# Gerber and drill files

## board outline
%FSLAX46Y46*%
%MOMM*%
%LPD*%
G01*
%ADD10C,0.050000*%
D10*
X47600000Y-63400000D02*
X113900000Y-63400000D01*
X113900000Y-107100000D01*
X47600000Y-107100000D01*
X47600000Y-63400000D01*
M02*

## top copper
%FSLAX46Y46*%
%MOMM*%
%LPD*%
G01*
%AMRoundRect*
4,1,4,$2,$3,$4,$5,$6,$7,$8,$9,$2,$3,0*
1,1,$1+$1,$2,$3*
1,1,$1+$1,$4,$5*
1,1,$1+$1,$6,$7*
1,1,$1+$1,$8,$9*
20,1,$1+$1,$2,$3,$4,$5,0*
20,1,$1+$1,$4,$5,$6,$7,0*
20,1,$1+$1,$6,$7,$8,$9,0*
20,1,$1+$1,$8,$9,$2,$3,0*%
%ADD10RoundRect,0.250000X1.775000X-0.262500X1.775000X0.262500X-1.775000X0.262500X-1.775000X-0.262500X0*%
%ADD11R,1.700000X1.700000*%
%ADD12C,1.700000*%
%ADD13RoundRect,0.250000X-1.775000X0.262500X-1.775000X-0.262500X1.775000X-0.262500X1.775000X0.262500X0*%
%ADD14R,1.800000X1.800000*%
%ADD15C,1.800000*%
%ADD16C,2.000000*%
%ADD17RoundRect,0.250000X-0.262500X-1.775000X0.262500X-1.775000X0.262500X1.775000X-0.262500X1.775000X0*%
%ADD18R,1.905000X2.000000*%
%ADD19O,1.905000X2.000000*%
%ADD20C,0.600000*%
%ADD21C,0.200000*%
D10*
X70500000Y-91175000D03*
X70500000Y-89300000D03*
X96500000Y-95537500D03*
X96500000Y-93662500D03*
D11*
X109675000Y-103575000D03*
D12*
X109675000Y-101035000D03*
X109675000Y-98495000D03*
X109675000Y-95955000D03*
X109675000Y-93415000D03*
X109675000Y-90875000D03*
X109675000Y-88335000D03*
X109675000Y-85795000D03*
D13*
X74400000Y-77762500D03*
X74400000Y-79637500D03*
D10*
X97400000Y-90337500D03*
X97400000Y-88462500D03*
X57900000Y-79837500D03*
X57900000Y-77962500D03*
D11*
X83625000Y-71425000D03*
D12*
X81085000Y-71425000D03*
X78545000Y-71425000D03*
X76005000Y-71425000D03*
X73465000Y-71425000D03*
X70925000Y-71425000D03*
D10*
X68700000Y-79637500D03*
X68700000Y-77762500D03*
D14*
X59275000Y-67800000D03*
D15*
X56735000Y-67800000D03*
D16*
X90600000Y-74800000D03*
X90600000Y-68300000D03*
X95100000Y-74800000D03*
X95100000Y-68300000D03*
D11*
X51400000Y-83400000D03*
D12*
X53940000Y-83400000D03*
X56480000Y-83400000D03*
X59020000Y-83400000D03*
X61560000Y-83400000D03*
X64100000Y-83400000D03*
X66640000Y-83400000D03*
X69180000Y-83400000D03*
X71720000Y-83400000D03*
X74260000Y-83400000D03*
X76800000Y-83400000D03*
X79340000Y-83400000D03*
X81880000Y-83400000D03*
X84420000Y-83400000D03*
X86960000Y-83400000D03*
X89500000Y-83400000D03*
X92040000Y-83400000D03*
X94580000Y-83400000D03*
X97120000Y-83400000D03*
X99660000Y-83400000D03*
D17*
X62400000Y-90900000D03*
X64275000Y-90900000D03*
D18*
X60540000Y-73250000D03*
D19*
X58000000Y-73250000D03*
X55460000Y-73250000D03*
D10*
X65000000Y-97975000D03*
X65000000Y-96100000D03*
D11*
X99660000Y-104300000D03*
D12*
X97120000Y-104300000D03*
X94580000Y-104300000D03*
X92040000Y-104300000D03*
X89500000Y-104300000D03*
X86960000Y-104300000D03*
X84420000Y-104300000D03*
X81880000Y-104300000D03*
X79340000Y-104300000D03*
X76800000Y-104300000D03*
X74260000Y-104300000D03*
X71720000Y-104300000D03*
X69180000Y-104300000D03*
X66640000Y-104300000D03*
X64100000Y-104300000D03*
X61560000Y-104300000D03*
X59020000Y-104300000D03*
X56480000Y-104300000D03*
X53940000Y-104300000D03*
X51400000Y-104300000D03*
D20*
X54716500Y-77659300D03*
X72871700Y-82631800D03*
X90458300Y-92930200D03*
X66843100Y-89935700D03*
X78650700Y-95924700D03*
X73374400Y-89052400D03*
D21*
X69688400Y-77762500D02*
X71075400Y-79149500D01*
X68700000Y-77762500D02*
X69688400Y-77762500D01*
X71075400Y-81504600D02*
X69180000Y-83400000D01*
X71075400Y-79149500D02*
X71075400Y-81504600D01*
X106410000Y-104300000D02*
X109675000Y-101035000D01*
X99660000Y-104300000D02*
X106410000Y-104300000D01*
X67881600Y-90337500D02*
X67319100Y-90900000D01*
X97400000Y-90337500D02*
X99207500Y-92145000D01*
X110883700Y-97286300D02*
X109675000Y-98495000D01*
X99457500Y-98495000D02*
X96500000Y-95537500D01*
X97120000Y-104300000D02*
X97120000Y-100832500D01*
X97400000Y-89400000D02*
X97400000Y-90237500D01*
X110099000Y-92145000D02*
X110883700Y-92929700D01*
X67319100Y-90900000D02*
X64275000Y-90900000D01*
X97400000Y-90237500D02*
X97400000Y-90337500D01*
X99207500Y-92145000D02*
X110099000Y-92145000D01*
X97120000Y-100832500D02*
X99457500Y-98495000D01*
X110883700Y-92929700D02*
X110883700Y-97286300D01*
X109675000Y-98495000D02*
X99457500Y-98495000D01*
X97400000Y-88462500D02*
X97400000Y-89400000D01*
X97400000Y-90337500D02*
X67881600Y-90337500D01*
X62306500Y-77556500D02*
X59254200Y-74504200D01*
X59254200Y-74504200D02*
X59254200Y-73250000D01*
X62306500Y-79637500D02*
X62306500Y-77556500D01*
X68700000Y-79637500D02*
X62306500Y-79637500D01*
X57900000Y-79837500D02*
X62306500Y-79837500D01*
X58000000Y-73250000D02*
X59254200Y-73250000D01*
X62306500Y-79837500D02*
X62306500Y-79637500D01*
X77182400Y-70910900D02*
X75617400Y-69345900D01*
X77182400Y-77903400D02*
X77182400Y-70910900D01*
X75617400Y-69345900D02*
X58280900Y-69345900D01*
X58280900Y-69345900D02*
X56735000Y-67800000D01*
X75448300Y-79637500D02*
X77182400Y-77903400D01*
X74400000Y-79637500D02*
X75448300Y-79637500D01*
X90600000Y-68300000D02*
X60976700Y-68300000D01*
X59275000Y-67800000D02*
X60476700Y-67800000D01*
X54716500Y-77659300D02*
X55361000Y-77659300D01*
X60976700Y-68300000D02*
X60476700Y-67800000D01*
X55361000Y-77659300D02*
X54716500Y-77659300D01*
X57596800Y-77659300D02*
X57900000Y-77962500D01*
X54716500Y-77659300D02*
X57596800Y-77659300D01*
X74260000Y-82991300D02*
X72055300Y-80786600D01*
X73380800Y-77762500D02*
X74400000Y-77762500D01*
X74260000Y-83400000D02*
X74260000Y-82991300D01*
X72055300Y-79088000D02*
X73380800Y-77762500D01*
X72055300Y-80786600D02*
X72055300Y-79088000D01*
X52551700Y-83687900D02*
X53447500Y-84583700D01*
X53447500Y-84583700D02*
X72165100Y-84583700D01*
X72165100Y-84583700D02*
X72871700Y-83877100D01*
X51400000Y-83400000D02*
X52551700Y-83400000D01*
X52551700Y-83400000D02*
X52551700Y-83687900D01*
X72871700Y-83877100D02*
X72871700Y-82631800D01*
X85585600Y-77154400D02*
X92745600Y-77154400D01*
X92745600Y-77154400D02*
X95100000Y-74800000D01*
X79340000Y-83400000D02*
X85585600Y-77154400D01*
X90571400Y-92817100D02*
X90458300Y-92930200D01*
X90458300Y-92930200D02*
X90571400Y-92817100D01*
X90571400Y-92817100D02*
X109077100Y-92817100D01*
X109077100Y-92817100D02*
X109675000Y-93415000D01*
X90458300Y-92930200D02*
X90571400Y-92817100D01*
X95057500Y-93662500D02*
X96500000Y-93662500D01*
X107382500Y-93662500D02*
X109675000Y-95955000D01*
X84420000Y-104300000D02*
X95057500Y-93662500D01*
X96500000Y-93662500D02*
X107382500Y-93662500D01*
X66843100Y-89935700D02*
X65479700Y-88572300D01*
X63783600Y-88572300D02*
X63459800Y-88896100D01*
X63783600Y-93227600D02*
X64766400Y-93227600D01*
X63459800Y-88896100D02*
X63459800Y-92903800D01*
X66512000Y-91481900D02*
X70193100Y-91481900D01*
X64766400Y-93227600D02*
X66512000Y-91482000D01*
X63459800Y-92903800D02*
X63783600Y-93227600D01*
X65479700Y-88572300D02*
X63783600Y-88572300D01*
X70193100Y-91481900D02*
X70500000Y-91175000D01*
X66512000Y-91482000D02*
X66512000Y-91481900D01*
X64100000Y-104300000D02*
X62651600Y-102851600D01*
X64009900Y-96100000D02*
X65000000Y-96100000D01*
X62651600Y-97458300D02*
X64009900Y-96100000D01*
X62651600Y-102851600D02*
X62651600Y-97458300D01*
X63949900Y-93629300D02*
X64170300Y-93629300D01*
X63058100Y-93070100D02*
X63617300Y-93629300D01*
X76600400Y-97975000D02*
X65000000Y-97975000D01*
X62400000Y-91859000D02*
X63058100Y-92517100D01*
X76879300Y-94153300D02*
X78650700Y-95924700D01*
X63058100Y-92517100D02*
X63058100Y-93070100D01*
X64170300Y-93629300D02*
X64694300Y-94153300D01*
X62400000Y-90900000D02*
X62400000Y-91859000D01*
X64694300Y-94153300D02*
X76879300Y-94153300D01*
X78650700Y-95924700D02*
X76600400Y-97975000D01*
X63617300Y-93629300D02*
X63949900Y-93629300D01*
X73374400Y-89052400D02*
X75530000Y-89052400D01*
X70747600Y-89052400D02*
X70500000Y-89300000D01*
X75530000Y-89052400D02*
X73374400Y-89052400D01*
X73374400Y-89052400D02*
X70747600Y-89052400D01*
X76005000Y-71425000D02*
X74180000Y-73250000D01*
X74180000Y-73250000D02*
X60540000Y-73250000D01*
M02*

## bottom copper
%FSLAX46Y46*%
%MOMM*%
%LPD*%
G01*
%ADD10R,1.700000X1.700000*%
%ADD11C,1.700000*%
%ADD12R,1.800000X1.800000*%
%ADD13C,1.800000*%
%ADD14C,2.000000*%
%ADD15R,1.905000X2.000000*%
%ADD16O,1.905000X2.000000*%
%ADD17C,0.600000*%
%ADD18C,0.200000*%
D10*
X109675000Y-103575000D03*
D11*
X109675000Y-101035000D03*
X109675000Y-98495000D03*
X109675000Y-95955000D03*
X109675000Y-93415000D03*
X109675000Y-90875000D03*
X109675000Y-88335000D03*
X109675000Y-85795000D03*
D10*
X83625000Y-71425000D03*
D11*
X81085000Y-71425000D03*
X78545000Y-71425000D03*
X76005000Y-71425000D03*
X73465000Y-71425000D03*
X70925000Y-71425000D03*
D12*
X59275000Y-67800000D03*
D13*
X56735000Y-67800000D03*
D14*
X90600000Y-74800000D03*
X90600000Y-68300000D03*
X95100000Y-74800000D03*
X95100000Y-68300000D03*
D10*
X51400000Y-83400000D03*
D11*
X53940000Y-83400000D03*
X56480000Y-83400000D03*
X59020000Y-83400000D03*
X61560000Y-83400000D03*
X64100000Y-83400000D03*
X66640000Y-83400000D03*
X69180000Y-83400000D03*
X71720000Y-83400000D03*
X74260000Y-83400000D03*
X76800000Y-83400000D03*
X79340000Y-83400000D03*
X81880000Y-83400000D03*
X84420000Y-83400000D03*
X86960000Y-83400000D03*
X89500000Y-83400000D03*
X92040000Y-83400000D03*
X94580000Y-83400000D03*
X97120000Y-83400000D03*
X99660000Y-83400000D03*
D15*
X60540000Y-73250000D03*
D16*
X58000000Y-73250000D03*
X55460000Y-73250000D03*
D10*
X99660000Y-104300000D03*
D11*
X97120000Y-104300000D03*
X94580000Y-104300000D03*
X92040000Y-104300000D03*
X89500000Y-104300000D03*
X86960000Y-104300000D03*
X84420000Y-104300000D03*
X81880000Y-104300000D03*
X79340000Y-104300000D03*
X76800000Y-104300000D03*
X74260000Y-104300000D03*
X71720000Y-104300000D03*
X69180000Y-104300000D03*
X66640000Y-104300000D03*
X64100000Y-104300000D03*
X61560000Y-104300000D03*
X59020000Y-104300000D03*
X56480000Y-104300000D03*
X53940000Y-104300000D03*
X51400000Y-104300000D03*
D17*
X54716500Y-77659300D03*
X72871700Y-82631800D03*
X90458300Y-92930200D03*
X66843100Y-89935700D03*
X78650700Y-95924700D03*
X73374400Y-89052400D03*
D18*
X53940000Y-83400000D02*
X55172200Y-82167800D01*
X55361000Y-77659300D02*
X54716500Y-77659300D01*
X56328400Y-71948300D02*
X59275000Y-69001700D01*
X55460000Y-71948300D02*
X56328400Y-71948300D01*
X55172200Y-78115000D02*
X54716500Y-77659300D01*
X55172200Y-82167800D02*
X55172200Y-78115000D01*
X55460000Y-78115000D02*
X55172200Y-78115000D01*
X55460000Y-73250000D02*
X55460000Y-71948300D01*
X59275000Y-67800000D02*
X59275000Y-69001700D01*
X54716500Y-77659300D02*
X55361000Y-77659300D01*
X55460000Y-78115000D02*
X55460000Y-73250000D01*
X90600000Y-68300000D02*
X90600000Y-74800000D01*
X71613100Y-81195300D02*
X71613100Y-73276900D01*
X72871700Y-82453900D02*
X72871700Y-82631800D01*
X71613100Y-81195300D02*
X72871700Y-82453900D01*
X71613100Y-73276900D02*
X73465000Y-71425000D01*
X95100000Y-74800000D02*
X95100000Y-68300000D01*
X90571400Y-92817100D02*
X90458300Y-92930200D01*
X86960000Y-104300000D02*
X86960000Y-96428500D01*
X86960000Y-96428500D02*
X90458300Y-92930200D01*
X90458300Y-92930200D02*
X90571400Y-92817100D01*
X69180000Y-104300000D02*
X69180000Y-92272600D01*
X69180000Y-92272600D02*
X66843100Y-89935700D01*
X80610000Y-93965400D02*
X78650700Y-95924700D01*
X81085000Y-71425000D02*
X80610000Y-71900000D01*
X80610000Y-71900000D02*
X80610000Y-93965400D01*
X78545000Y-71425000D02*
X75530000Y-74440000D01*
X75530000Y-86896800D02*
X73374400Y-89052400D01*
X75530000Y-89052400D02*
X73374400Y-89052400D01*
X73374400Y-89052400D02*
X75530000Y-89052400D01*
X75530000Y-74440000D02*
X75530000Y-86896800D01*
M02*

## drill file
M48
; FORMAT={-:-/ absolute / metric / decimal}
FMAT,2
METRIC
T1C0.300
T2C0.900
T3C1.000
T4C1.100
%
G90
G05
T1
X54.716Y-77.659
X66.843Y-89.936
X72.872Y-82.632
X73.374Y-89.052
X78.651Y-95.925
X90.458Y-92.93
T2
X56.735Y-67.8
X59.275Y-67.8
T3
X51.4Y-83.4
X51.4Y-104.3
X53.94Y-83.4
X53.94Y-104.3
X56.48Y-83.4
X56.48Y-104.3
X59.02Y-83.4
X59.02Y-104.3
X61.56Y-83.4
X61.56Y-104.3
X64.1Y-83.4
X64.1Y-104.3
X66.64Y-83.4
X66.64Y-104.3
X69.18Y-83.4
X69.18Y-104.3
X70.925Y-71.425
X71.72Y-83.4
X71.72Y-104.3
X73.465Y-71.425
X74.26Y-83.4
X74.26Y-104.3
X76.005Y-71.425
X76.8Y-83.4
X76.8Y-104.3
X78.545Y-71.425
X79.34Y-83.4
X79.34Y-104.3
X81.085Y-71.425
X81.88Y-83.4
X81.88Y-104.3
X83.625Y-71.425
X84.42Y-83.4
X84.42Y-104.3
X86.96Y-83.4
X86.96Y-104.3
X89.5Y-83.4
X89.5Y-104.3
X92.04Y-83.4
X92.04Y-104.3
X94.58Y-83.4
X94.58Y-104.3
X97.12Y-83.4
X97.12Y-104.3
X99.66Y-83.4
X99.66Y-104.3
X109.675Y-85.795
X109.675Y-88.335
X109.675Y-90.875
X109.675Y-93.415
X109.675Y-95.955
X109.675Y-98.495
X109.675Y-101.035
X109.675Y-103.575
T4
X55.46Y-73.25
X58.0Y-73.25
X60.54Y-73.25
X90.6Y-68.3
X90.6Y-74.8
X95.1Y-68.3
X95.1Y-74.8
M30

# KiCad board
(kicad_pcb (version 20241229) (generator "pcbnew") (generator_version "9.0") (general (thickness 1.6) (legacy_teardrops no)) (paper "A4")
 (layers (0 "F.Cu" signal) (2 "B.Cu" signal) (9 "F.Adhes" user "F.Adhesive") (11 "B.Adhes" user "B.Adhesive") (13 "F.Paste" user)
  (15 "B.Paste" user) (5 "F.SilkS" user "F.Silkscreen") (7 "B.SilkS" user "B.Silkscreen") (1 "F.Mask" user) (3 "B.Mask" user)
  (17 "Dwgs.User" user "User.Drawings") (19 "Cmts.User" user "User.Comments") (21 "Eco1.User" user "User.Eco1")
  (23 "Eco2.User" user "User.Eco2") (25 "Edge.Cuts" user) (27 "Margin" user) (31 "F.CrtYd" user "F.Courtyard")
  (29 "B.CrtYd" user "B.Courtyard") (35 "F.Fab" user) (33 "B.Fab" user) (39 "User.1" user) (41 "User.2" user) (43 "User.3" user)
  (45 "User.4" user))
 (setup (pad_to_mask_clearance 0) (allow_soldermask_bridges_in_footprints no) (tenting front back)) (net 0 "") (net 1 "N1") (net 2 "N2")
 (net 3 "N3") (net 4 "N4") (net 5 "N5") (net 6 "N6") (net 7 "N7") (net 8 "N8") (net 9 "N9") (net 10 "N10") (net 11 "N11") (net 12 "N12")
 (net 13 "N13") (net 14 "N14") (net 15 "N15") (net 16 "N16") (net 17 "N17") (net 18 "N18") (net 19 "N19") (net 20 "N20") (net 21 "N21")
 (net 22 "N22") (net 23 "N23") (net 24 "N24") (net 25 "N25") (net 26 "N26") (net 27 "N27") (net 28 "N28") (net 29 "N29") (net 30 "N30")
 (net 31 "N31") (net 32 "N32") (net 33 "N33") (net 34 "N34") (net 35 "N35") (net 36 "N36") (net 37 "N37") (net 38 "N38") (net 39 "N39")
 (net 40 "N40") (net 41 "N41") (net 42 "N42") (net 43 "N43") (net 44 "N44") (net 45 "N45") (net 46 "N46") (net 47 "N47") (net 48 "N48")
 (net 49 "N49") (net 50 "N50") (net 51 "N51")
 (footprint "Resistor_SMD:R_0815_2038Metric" (layer "F.Cu") (at 70.5 90.2375 90)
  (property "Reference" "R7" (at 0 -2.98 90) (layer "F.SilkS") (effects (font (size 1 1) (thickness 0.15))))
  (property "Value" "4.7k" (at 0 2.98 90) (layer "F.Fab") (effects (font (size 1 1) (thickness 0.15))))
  (pad "1" smd roundrect (at -0.9375 0 90) (size 1.025 4.05) (layers "F.Cu" "F.Mask" "F.Paste") (roundrect_rratio 0.243902) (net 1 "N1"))
  (pad "2" smd roundrect (at 0.9375 0 90) (size 1.025 4.05) (layers "F.Cu" "F.Mask" "F.Paste") (roundrect_rratio 0.243902) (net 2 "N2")))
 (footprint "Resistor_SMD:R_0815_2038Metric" (layer "F.Cu") (at 96.5 94.6 90)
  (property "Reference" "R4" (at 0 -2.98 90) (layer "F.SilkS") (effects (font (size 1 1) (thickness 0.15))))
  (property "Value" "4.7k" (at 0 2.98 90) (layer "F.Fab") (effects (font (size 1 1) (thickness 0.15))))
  (pad "1" smd roundrect (at -0.9375 0 90) (size 1.025 4.05) (layers "F.Cu" "F.Mask" "F.Paste") (roundrect_rratio 0.243902) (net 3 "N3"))
  (pad "2" smd roundrect (at 0.9375 0 90) (size 1.025 4.05) (layers "F.Cu" "F.Mask" "F.Paste") (roundrect_rratio 0.243902) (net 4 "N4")))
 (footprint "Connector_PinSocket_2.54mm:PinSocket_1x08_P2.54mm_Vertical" (layer "F.Cu") (at 109.675 103.575 180)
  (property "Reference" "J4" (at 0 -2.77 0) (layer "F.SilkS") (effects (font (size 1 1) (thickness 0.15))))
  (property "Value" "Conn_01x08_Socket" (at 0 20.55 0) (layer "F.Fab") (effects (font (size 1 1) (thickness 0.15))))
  (pad "1" thru_hole rect (at 0 0 180) (size 1.7 1.7) (drill 1) (layers "*.Cu" "*.Mask") (remove_unused_layers no) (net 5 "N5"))
  (pad "2" thru_hole circle (at 0 2.54 180) (size 1.7 1.7) (drill 1) (layers "*.Cu" "*.Mask") (remove_unused_layers no) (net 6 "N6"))
  (pad "3" thru_hole circle (at 0 5.08 180) (size 1.7 1.7) (drill 1) (layers "*.Cu" "*.Mask") (remove_unused_layers no) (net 3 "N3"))
  (pad "4" thru_hole circle (at 0 7.62 180) (size 1.7 1.7) (drill 1) (layers "*.Cu" "*.Mask") (remove_unused_layers no) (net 4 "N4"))
  (pad "5" thru_hole circle (at 0 10.16 180) (size 1.7 1.7) (drill 1) (layers "*.Cu" "*.Mask") (remove_unused_layers no) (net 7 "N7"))
  (pad "6" thru_hole circle (at 0 12.7 180) (size 1.7 1.7) (drill 1) (layers "*.Cu" "*.Mask") (remove_unused_layers no) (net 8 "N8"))
  (pad "7" thru_hole circle (at 0 15.24 180) (size 1.7 1.7) (drill 1) (layers "*.Cu" "*.Mask") (remove_unused_layers no) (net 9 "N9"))
  (pad "8" thru_hole circle (at 0 17.78 180) (size 1.7 1.7) (drill 1) (layers "*.Cu" "*.Mask") (remove_unused_layers no) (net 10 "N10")))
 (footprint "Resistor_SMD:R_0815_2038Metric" (layer "F.Cu") (at 74.4 78.7 -90)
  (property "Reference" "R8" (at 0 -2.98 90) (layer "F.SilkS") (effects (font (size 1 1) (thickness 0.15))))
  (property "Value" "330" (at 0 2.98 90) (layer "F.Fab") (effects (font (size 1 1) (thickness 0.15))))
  (pad "1" smd roundrect (at -0.9375 0 270) (size 1.025 4.05) (layers "F.Cu" "F.Mask" "F.Paste") (roundrect_rratio 0.243902) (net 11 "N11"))
  (pad "2" smd roundrect (at 0.9375 0 270) (size 1.025 4.05) (layers "F.Cu" "F.Mask" "F.Paste") (roundrect_rratio 0.243902) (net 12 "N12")))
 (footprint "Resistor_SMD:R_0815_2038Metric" (layer "F.Cu") (at 97.4 89.4 90)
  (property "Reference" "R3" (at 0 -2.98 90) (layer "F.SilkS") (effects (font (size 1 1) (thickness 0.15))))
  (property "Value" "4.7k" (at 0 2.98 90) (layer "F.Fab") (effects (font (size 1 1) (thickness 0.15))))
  (pad "1" smd roundrect (at -0.9375 0 90) (size 1.025 4.05) (layers "F.Cu" "F.Mask" "F.Paste") (roundrect_rratio 0.243902) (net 3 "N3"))
  (pad "2" smd roundrect (at 0.9375 0 90) (size 1.025 4.05) (layers "F.Cu" "F.Mask" "F.Paste") (roundrect_rratio 0.243902) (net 3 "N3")))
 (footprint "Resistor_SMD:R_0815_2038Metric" (layer "F.Cu") (at 57.9 78.9 90)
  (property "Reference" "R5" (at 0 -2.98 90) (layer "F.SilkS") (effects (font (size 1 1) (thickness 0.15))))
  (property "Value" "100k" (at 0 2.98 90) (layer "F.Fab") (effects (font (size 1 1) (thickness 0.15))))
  (pad "1" smd roundrect (at -0.9375 0 90) (size 1.025 4.05) (layers "F.Cu" "F.Mask" "F.Paste") (roundrect_rratio 0.243902) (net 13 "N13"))
  (pad "2" smd roundrect (at 0.9375 0 90) (size 1.025 4.05) (layers "F.Cu" "F.Mask" "F.Paste") (roundrect_rratio 0.243902) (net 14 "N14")))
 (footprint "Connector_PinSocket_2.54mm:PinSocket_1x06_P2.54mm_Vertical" (layer "F.Cu") (at 83.625 71.425 -90)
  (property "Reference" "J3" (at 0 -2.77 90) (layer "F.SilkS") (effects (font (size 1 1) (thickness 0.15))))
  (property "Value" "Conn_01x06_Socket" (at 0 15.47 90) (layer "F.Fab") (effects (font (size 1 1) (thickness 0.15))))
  (pad "1" thru_hole rect (at 0 0 270) (size 1.7 1.7) (drill 1) (layers "*.Cu" "*.Mask") (remove_unused_layers no) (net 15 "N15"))
  (pad "2" thru_hole circle (at 0 2.54 270) (size 1.7 1.7) (drill 1) (layers "*.Cu" "*.Mask") (remove_unused_layers no) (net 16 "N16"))
  (pad "3" thru_hole circle (at 0 5.08 270) (size 1.7 1.7) (drill 1) (layers "*.Cu" "*.Mask") (remove_unused_layers no) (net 2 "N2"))
  (pad "4" thru_hole circle (at 0 7.62 270) (size 1.7 1.7) (drill 1) (layers "*.Cu" "*.Mask") (remove_unused_layers no) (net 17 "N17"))
  (pad "5" thru_hole circle (at 0 10.16 270) (size 1.7 1.7) (drill 1) (layers "*.Cu" "*.Mask") (remove_unused_layers no) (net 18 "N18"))
  (pad "6" thru_hole circle (at 0 12.7 270) (size 1.7 1.7) (drill 1) (layers "*.Cu" "*.Mask") (remove_unused_layers no) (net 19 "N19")))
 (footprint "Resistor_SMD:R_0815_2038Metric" (layer "F.Cu") (at 68.7 78.7 90)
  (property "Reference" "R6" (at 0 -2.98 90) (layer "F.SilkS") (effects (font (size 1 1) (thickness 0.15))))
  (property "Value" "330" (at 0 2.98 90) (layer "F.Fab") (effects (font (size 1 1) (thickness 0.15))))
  (pad "1" smd roundrect (at -0.9375 0 90) (size 1.025 4.05) (layers "F.Cu" "F.Mask" "F.Paste") (roundrect_rratio 0.243902) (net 13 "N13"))
  (pad "2" smd roundrect (at 0.9375 0 90) (size 1.025 4.05) (layers "F.Cu" "F.Mask" "F.Paste") (roundrect_rratio 0.243902) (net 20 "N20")))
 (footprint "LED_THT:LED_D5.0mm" (layer "F.Cu") (at 59.275 67.8 180)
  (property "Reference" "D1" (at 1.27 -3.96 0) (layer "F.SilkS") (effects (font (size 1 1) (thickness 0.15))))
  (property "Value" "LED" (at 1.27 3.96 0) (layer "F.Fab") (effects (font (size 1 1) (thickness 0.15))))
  (pad "1" thru_hole rect (at 0 0 180) (size 1.8 1.8) (drill 0.9) (layers "*.Cu" "*.Mask") (remove_unused_layers no) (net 14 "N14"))
  (pad "2" thru_hole circle (at 2.54 0 180) (size 1.8 1.8) (drill 0.9) (layers "*.Cu" "*.Mask") (remove_unused_layers no) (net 12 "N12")))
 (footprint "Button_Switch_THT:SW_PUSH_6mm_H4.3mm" (layer "F.Cu") (at 90.6 74.8 90)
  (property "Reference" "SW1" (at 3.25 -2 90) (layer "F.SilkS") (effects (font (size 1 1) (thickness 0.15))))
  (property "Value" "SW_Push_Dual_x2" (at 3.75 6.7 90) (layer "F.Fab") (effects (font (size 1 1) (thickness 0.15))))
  (pad "1" thru_hole circle (at 0 0 180) (size 2 2) (drill 1.1) (layers "*.Cu" "*.Mask") (remove_unused_layers no) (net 14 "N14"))
  (pad "1" thru_hole circle (at 6.5 0 180) (size 2 2) (drill 1.1) (layers "*.Cu" "*.Mask") (remove_unused_layers no) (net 14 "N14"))
  (pad "2" thru_hole circle (at 0 4.5 180) (size 2 2) (drill 1.1) (layers "*.Cu" "*.Mask") (remove_unused_layers no) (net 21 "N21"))
  (pad "2" thru_hole circle (at 6.5 4.5 180) (size 2 2) (drill 1.1) (layers "*.Cu" "*.Mask") (remove_unused_layers no) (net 21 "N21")))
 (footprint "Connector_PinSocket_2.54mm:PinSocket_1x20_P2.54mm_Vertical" (layer "F.Cu") (at 51.4 83.4 90)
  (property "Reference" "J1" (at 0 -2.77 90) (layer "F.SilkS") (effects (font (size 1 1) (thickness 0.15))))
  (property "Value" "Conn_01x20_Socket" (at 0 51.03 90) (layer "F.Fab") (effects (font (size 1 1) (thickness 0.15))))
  (pad "1" thru_hole rect (at 0 0 90) (size 1.7 1.7) (drill 1) (layers "*.Cu" "*.Mask") (remove_unused_layers no) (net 18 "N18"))
  (pad "2" thru_hole circle (at 0 2.54 90) (size 1.7 1.7) (drill 1) (layers "*.Cu" "*.Mask") (remove_unused_layers no) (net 14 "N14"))
  (pad "3" thru_hole circle (at 0 5.08 90) (size 1.7 1.7) (drill 1) (layers "*.Cu" "*.Mask") (remove_unused_layers no) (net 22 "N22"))
  (pad "4" thru_hole circle (at 0 7.62 90) (size 1.7 1.7) (drill 1) (layers "*.Cu" "*.Mask") (remove_unused_layers no) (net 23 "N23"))
  (pad "5" thru_hole circle (at 0 10.16 90) (size 1.7 1.7) (drill 1) (layers "*.Cu" "*.Mask") (remove_unused_layers no) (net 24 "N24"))
  (pad "6" thru_hole circle (at 0 12.7 90) (size 1.7 1.7) (drill 1) (layers "*.Cu" "*.Mask") (remove_unused_layers no) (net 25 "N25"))
  (pad "7" thru_hole circle (at 0 15.24 90) (size 1.7 1.7) (drill 1) (layers "*.Cu" "*.Mask") (remove_unused_layers no) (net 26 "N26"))
  (pad "8" thru_hole circle (at 0 17.78 90) (size 1.7 1.7) (drill 1) (layers "*.Cu" "*.Mask") (remove_unused_layers no) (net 20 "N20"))
  (pad "9" thru_hole circle (at 0 20.32 90) (size 1.7 1.7) (drill 1) (layers "*.Cu" "*.Mask") (remove_unused_layers no) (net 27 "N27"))
  (pad "10" thru_hole circle (at 0 22.86 90) (size 1.7 1.7) (drill 1) (layers "*.Cu" "*.Mask") (remove_unused_layers no) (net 11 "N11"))
  (pad "11" thru_hole circle (at 0 25.4 90) (size 1.7 1.7) (drill 1) (layers "*.Cu" "*.Mask") (remove_unused_layers no) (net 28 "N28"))
  (pad "12" thru_hole circle (at 0 27.94 90) (size 1.7 1.7) (drill 1) (layers "*.Cu" "*.Mask") (remove_unused_layers no) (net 21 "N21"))
  (pad "13" thru_hole circle (at 0 30.48 90) (size 1.7 1.7) (drill 1) (layers "*.Cu" "*.Mask") (remove_unused_layers no) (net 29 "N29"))
  (pad "14" thru_hole circle (at 0 33.02 90) (size 1.7 1.7) (drill 1) (layers "*.Cu" "*.Mask") (remove_unused_layers no) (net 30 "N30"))
  (pad "15" thru_hole circle (at 0 35.56 90) (size 1.7 1.7) (drill 1) (layers "*.Cu" "*.Mask") (remove_unused_layers no) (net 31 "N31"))
  (pad "16" thru_hole circle (at 0 38.1 90) (size 1.7 1.7) (drill 1) (layers "*.Cu" "*.Mask") (remove_unused_layers no) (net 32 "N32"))
  (pad "17" thru_hole circle (at 0 40.64 90) (size 1.7 1.7) (drill 1) (layers "*.Cu" "*.Mask") (remove_unused_layers no) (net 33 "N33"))
  (pad "18" thru_hole circle (at 0 43.18 90) (size 1.7 1.7) (drill 1) (layers "*.Cu" "*.Mask") (remove_unused_layers no) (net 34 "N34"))
  (pad "19" thru_hole circle (at 0 45.72 90) (size 1.7 1.7) (drill 1) (layers "*.Cu" "*.Mask") (remove_unused_layers no) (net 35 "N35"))
  (pad "20" thru_hole circle (at 0 48.26 90) (size 1.7 1.7) (drill 1) (layers "*.Cu" "*.Mask") (remove_unused_layers no) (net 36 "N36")))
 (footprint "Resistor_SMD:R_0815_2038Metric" (layer "F.Cu") (at 63.3375 90.9)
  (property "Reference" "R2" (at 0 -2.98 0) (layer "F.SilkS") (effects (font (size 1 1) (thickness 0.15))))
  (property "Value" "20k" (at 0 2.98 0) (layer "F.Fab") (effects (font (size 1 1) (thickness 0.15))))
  (pad "1" smd roundrect (at -0.9375 0) (size 1.025 4.05) (layers "F.Cu" "F.Mask" "F.Paste") (roundrect_rratio 0.243902) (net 16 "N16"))
  (pad "2" smd roundrect (at 0.9375 0) (size 1.025 4.05) (layers "F.Cu" "F.Mask" "F.Paste") (roundrect_rratio 0.243902) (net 3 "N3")))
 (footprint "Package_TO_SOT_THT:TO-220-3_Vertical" (layer "F.Cu") (at 60.54 73.25 180)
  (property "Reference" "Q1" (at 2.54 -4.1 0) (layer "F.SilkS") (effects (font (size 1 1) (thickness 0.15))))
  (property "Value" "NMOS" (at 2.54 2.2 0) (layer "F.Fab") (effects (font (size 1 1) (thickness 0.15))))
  (pad "1" thru_hole rect (at 0 0 180) (size 1.905 2) (drill 1.1) (layers "*.Cu" "*.Mask") (remove_unused_layers no) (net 17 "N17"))
  (pad "2" thru_hole oval (at 2.54 0 180) (size 1.905 2) (drill 1.1) (layers "*.Cu" "*.Mask") (remove_unused_layers no) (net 13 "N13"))
  (pad "3" thru_hole oval (at 5.08 0 180) (size 1.905 2) (drill 1.1) (layers "*.Cu" "*.Mask") (remove_unused_layers no) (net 14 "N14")))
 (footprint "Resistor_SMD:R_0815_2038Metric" (layer "F.Cu") (at 65 97.0375 90)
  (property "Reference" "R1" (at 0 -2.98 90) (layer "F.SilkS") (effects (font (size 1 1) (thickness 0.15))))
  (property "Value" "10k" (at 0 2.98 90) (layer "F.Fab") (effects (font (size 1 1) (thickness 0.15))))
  (pad "1" smd roundrect (at -0.9375 0 90) (size 1.025 4.05) (layers "F.Cu" "F.Mask" "F.Paste") (roundrect_rratio 0.243902) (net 16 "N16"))
  (pad "2" smd roundrect (at 0.9375 0 90) (size 1.025 4.05) (layers "F.Cu" "F.Mask" "F.Paste") (roundrect_rratio 0.243902) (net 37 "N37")))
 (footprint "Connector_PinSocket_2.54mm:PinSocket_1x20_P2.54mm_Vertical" (layer "F.Cu") (at 99.66 104.3 -90)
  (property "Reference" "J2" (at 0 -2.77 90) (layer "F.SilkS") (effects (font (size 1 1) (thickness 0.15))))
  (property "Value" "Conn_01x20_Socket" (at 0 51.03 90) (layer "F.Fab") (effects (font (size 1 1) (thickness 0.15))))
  (pad "1" thru_hole rect (at 0 0 270) (size 1.7 1.7) (drill 1) (layers "*.Cu" "*.Mask") (remove_unused_layers no) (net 6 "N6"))
  (pad "2" thru_hole circle (at 0 2.54 270) (size 1.7 1.7) (drill 1) (layers "*.Cu" "*.Mask") (remove_unused_layers no) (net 3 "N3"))
  (pad "3" thru_hole circle (at 0 5.08 270) (size 1.7 1.7) (drill 1) (layers "*.Cu" "*.Mask") (remove_unused_layers no) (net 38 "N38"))
  (pad "4" thru_hole circle (at 0 7.62 270) (size 1.7 1.7) (drill 1) (layers "*.Cu" "*.Mask") (remove_unused_layers no) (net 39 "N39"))
  (pad "5" thru_hole circle (at 0 10.16 270) (size 1.7 1.7) (drill 1) (layers "*.Cu" "*.Mask") (remove_unused_layers no) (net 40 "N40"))
  (pad "6" thru_hole circle (at 0 12.7 270) (size 1.7 1.7) (drill 1) (layers "*.Cu" "*.Mask") (remove_unused_layers no) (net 7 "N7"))
  (pad "7" thru_hole circle (at 0 15.24 270) (size 1.7 1.7) (drill 1) (layers "*.Cu" "*.Mask") (remove_unused_layers no) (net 4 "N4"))
  (pad "8" thru_hole circle (at 0 17.78 270) (size 1.7 1.7) (drill 1) (layers "*.Cu" "*.Mask") (remove_unused_layers no) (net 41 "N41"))
  (pad "9" thru_hole circle (at 0 20.32 270) (size 1.7 1.7) (drill 1) (layers "*.Cu" "*.Mask") (remove_unused_layers no) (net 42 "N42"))
  (pad "10" thru_hole circle (at 0 22.86 270) (size 1.7 1.7) (drill 1) (layers "*.Cu" "*.Mask") (remove_unused_layers no) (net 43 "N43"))
  (pad "11" thru_hole circle (at 0 25.4 270) (size 1.7 1.7) (drill 1) (layers "*.Cu" "*.Mask") (remove_unused_layers no) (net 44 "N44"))
  (pad "12" thru_hole circle (at 0 27.94 270) (size 1.7 1.7) (drill 1) (layers "*.Cu" "*.Mask") (remove_unused_layers no) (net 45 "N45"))
  (pad "13" thru_hole circle (at 0 30.48 270) (size 1.7 1.7) (drill 1) (layers "*.Cu" "*.Mask") (remove_unused_layers no) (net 1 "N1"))
  (pad "14" thru_hole circle (at 0 33.02 270) (size 1.7 1.7) (drill 1) (layers "*.Cu" "*.Mask") (remove_unused_layers no) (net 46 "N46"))
  (pad "15" thru_hole circle (at 0 35.56 270) (size 1.7 1.7) (drill 1) (layers "*.Cu" "*.Mask") (remove_unused_layers no) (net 37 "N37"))
  (pad "16" thru_hole circle (at 0 38.1 270) (size 1.7 1.7) (drill 1) (layers "*.Cu" "*.Mask") (remove_unused_layers no) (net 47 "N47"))
  (pad "17" thru_hole circle (at 0 40.64 270) (size 1.7 1.7) (drill 1) (layers "*.Cu" "*.Mask") (remove_unused_layers no) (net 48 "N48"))
  (pad "18" thru_hole circle (at 0 43.18 270) (size 1.7 1.7) (drill 1) (layers "*.Cu" "*.Mask") (remove_unused_layers no) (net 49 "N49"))
  (pad "19" thru_hole circle (at 0 45.72 270) (size 1.7 1.7) (drill 1) (layers "*.Cu" "*.Mask") (remove_unused_layers no) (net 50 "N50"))
  (pad "20" thru_hole circle (at 0 48.26 270) (size 1.7 1.7) (drill 1) (layers "*.Cu" "*.Mask") (remove_unused_layers no) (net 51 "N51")))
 (gr_rect (start 47.6 63.4) (end 113.9 107.1) (stroke (width 0.05) (type default)) (fill no) (layer "Edge.Cuts"))
 (segment (start 69.6884 77.7625) (end 71.0754 79.1495) (width 0.2) (layer "F.Cu") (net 20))
 (segment (start 68.7 77.7625) (end 69.6884 77.7625) (width 0.2) (layer "F.Cu") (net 20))
 (segment (start 71.0754 81.5046) (end 69.18 83.4) (width 0.2) (layer "F.Cu") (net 20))
 (segment (start 71.0754 79.1495) (end 71.0754 81.5046) (width 0.2) (layer "F.Cu") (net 20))
 (segment (start 106.41 104.3) (end 109.675 101.035) (width 0.2) (layer "F.Cu") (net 6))
 (segment (start 99.66 104.3) (end 106.41 104.3) (width 0.2) (layer "F.Cu") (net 6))
 (segment (start 67.8816 90.3375) (end 67.3191 90.9) (width 0.2) (layer "F.Cu") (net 3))
 (segment (start 97.4 90.3375) (end 99.2075 92.145) (width 0.2) (layer "F.Cu") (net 3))
 (segment (start 110.8837 97.2863) (end 109.675 98.495) (width 0.2) (layer "F.Cu") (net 3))
 (segment (start 99.4575 98.495) (end 96.5 95.5375) (width 0.2) (layer "F.Cu") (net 3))
 (segment (start 97.12 104.3) (end 97.12 100.8325) (width 0.2) (layer "F.Cu") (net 3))
 (segment (start 97.4 89.4) (end 97.4 90.2375) (width 0.2) (layer "F.Cu") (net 3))
 (segment (start 110.099 92.145) (end 110.8837 92.9297) (width 0.2) (layer "F.Cu") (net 3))
 (segment (start 67.3191 90.9) (end 64.275 90.9) (width 0.2) (layer "F.Cu") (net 3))
 (segment (start 97.4 90.2375) (end 97.4 90.3375) (width 0.2) (layer "F.Cu") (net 3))
 (segment (start 99.2075 92.145) (end 110.099 92.145) (width 0.2) (layer "F.Cu") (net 3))
 (segment (start 97.12 100.8325) (end 99.4575 98.495) (width 0.2) (layer "F.Cu") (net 3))
 (segment (start 110.8837 92.9297) (end 110.8837 97.2863) (width 0.2) (layer "F.Cu") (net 3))
 (segment (start 109.675 98.495) (end 99.4575 98.495) (width 0.2) (layer "F.Cu") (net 3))
 (segment (start 97.4 88.4625) (end 97.4 89.4) (width 0.2) (layer "F.Cu") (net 3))
 (segment (start 97.4 90.3375) (end 67.8816 90.3375) (width 0.2) (layer "F.Cu") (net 3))
 (segment (start 62.3065 77.5565) (end 59.2542 74.5042) (width 0.2) (layer "F.Cu") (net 13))
 (segment (start 59.2542 74.5042) (end 59.2542 73.25) (width 0.2) (layer "F.Cu") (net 13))
 (segment (start 62.3065 79.6375) (end 62.3065 77.5565) (width 0.2) (layer "F.Cu") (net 13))
 (segment (start 68.7 79.6375) (end 62.3065 79.6375) (width 0.2) (layer "F.Cu") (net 13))
 (segment (start 57.9 79.8375) (end 62.3065 79.8375) (width 0.2) (layer "F.Cu") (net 13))
 (segment (start 58 73.25) (end 59.2542 73.25) (width 0.2) (layer "F.Cu") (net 13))
 (segment (start 62.3065 79.8375) (end 62.3065 79.6375) (width 0.2) (layer "F.Cu") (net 13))
 (segment (start 77.1824 70.9109) (end 75.6174 69.3459) (width 0.2) (layer "F.Cu") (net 12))
 (segment (start 77.1824 77.9034) (end 77.1824 70.9109) (width 0.2) (layer "F.Cu") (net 12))
 (segment (start 75.6174 69.3459) (end 58.2809 69.3459) (width 0.2) (layer "F.Cu") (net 12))
 (segment (start 58.2809 69.3459) (end 56.735 67.8) (width 0.2) (layer "F.Cu") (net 12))
 (segment (start 75.4483 79.6375) (end 77.1824 77.9034) (width 0.2) (layer "F.Cu") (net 12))
 (segment (start 74.4 79.6375) (end 75.4483 79.6375) (width 0.2) (layer "F.Cu") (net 12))
 (segment (start 90.6 68.3) (end 60.9767 68.3) (width 0.2) (layer "F.Cu") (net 14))
 (segment (start 59.275 67.8) (end 60.4767 67.8) (width 0.2) (layer "F.Cu") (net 14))
 (segment (start 54.7165 77.6593) (end 55.361 77.6593) (width 0.2) (layer "F.Cu") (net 14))
 (segment (start 60.9767 68.3) (end 60.4767 67.8) (width 0.2) (layer "F.Cu") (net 14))
 (segment (start 55.361 77.6593) (end 54.7165 77.6593) (width 0.2) (layer "F.Cu") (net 14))
 (segment (start 57.5968 77.6593) (end 57.9 77.9625) (width 0.2) (layer "F.Cu") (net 14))
 (segment (start 54.7165 77.6593) (end 57.5968 77.6593) (width 0.2) (layer "F.Cu") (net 14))
 (via (at 54.7165 77.6593) (size 0.6) (drill 0.3) (layers "F.Cu" "B.Cu") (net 14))
 (segment (start 53.94 83.4) (end 55.1722 82.1678) (width 0.2) (layer "B.Cu") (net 14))
 (segment (start 55.361 77.6593) (end 54.7165 77.6593) (width 0.2) (layer "B.Cu") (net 14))
 (segment (start 56.3284 71.9483) (end 59.275 69.0017) (width 0.2) (layer "B.Cu") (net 14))
 (segment (start 55.46 71.9483) (end 56.3284 71.9483) (width 0.2) (layer "B.Cu") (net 14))
 (segment (start 55.1722 78.115) (end 54.7165 77.6593) (width 0.2) (layer "B.Cu") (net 14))
 (segment (start 55.1722 82.1678) (end 55.1722 78.115) (width 0.2) (layer "B.Cu") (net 14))
 (segment (start 55.46 78.115) (end 55.1722 78.115) (width 0.2) (layer "B.Cu") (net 14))
 (segment (start 55.46 73.25) (end 55.46 71.9483) (width 0.2) (layer "B.Cu") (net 14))
 (segment (start 59.275 67.8) (end 59.275 69.0017) (width 0.2) (layer "B.Cu") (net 14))
 (segment (start 54.7165 77.6593) (end 55.361 77.6593) (width 0.2) (layer "B.Cu") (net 14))
 (segment (start 55.46 78.115) (end 55.46 73.25) (width 0.2) (layer "B.Cu") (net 14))
 (segment (start 90.6 68.3) (end 90.6 74.8) (width 0.2) (layer "B.Cu") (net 14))
 (segment (start 74.26 82.9913) (end 72.0553 80.7866) (width 0.2) (layer "F.Cu") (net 11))
 (segment (start 73.3808 77.7625) (end 74.4 77.7625) (width 0.2) (layer "F.Cu") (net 11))
 (segment (start 74.26 83.4) (end 74.26 82.9913) (width 0.2) (layer "F.Cu") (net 11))
 (segment (start 72.0553 79.088) (end 73.3808 77.7625) (width 0.2) (layer "F.Cu") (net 11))
 (segment (start 72.0553 80.7866) (end 72.0553 79.088) (width 0.2) (layer "F.Cu") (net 11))
 (segment (start 52.5517 83.6879) (end 53.4475 84.5837) (width 0.2) (layer "F.Cu") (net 18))
 (segment (start 53.4475 84.5837) (end 72.1651 84.5837) (width 0.2) (layer "F.Cu") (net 18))
 (segment (start 72.1651 84.5837) (end 72.8717 83.8771) (width 0.2) (layer "F.Cu") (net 18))
 (segment (start 51.4 83.4) (end 52.5517 83.4) (width 0.2) (layer "F.Cu") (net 18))
 (segment (start 52.5517 83.4) (end 52.5517 83.6879) (width 0.2) (layer "F.Cu") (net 18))
 (segment (start 72.8717 83.8771) (end 72.8717 82.6318) (width 0.2) (layer "F.Cu") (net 18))
 (via (at 72.8717 82.6318) (size 0.6) (drill 0.3) (layers "F.Cu" "B.Cu") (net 18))
 (segment (start 71.6131 81.1953) (end 71.6131 73.2769) (width 0.2) (layer "B.Cu") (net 18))
 (segment (start 72.8717 82.4539) (end 72.8717 82.6318) (width 0.2) (layer "B.Cu") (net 18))
 (segment (start 71.6131 81.1953) (end 72.8717 82.4539) (width 0.2) (layer "B.Cu") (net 18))
 (segment (start 71.6131 73.2769) (end 73.465 71.425) (width 0.2) (layer "B.Cu") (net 18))
 (segment (start 85.5856 77.1544) (end 92.7456 77.1544) (width 0.2) (layer "F.Cu") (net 21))
 (segment (start 92.7456 77.1544) (end 95.1 74.8) (width 0.2) (layer "F.Cu") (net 21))
 (segment (start 79.34 83.4) (end 85.5856 77.1544) (width 0.2) (layer "F.Cu") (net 21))
 (segment (start 95.1 74.8) (end 95.1 68.3) (width 0.2) (layer "B.Cu") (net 21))
 (segment (start 90.5714 92.8171) (end 90.4583 92.9302) (width 0.2) (layer "F.Cu") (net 7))
 (segment (start 90.4583 92.9302) (end 90.5714 92.8171) (width 0.2) (layer "F.Cu") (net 7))
 (segment (start 90.5714 92.8171) (end 109.0771 92.8171) (width 0.2) (layer "F.Cu") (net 7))
 (segment (start 109.0771 92.8171) (end 109.675 93.415) (width 0.2) (layer "F.Cu") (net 7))
 (segment (start 90.4583 92.9302) (end 90.5714 92.8171) (width 0.2) (layer "F.Cu") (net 7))
 (via (at 90.4583 92.9302) (size 0.6) (drill 0.3) (layers "F.Cu" "B.Cu") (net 7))
 (segment (start 90.5714 92.8171) (end 90.4583 92.9302) (width 0.2) (layer "B.Cu") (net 7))
 (segment (start 86.96 104.3) (end 86.96 96.4285) (width 0.2) (layer "B.Cu") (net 7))
 (segment (start 86.96 96.4285) (end 90.4583 92.9302) (width 0.2) (layer "B.Cu") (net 7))
 (segment (start 90.4583 92.9302) (end 90.5714 92.8171) (width 0.2) (layer "B.Cu") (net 7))
 (segment (start 95.0575 93.6625) (end 96.5 93.6625) (width 0.2) (layer "F.Cu") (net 4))
 (segment (start 107.3825 93.6625) (end 109.675 95.955) (width 0.2) (layer "F.Cu") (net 4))
 (segment (start 84.42 104.3) (end 95.0575 93.6625) (width 0.2) (layer "F.Cu") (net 4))
 (segment (start 96.5 93.6625) (end 107.3825 93.6625) (width 0.2) (layer "F.Cu") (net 4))
 (segment (start 66.8431 89.9357) (end 65.4797 88.5723) (width 0.2) (layer "F.Cu") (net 1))
 (segment (start 63.7836 88.5723) (end 63.4598 88.8961) (width 0.2) (layer "F.Cu") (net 1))
 (segment (start 63.7836 93.2276) (end 64.7664 93.2276) (width 0.2) (layer "F.Cu") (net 1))
 (segment (start 63.4598 88.8961) (end 63.4598 92.9038) (width 0.2) (layer "F.Cu") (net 1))
 (segment (start 66.512 91.4819) (end 70.1931 91.4819) (width 0.2) (layer "F.Cu") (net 1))
 (segment (start 64.7664 93.2276) (end 66.512 91.482) (width 0.2) (layer "F.Cu") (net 1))
 (segment (start 63.4598 92.9038) (end 63.7836 93.2276) (width 0.2) (layer "F.Cu") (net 1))
 (segment (start 65.4797 88.5723) (end 63.7836 88.5723) (width 0.2) (layer "F.Cu") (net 1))
 (segment (start 70.1931 91.4819) (end 70.5 91.175) (width 0.2) (layer "F.Cu") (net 1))
 (segment (start 66.512 91.482) (end 66.512 91.4819) (width 0.2) (layer "F.Cu") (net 1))
 (via (at 66.8431 89.9357) (size 0.6) (drill 0.3) (layers "F.Cu" "B.Cu") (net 1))
 (segment (start 69.18 104.3) (end 69.18 92.2726) (width 0.2) (layer "B.Cu") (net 1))
 (segment (start 69.18 92.2726) (end 66.8431 89.9357) (width 0.2) (layer "B.Cu") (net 1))
 (segment (start 64.1 104.3) (end 62.6516 102.8516) (width 0.2) (layer "F.Cu") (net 37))
 (segment (start 64.0099 96.1) (end 65 96.1) (width 0.2) (layer "F.Cu") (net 37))
 (segment (start 62.6516 97.4583) (end 64.0099 96.1) (width 0.2) (layer "F.Cu") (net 37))
 (segment (start 62.6516 102.8516) (end 62.6516 97.4583) (width 0.2) (layer "F.Cu") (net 37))
 (segment (start 63.9499 93.6293) (end 64.1703 93.6293) (width 0.2) (layer "F.Cu") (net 16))
 (segment (start 63.0581 93.0701) (end 63.6173 93.6293) (width 0.2) (layer "F.Cu") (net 16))
 (segment (start 76.6004 97.975) (end 65 97.975) (width 0.2) (layer "F.Cu") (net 16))
 (segment (start 62.4 91.859) (end 63.0581 92.5171) (width 0.2) (layer "F.Cu") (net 16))
 (segment (start 76.8793 94.1533) (end 78.6507 95.9247) (width 0.2) (layer "F.Cu") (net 16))
 (segment (start 63.0581 92.5171) (end 63.0581 93.0701) (width 0.2) (layer "F.Cu") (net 16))
 (segment (start 64.1703 93.6293) (end 64.6943 94.1533) (width 0.2) (layer "F.Cu") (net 16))
 (segment (start 62.4 90.9) (end 62.4 91.859) (width 0.2) (layer "F.Cu") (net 16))
 (segment (start 64.6943 94.1533) (end 76.8793 94.1533) (width 0.2) (layer "F.Cu") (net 16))
 (segment (start 78.6507 95.9247) (end 76.6004 97.975) (width 0.2) (layer "F.Cu") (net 16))
 (segment (start 63.6173 93.6293) (end 63.9499 93.6293) (width 0.2) (layer "F.Cu") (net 16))
 (via (at 78.6507 95.9247) (size 0.6) (drill 0.3) (layers "F.Cu" "B.Cu") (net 16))
 (segment (start 80.61 93.9654) (end 78.6507 95.9247) (width 0.2) (layer "B.Cu") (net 16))
 (segment (start 81.085 71.425) (end 80.61 71.9) (width 0.2) (layer "B.Cu") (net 16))
 (segment (start 80.61 71.9) (end 80.61 93.9654) (width 0.2) (layer "B.Cu") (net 16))
 (segment (start 73.3744 89.0524) (end 75.53 89.0524) (width 0.2) (layer "F.Cu") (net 2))
 (segment (start 70.7476 89.0524) (end 70.5 89.3) (width 0.2) (layer "F.Cu") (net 2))
 (segment (start 75.53 89.0524) (end 73.3744 89.0524) (width 0.2) (layer "F.Cu") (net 2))
 (segment (start 73.3744 89.0524) (end 70.7476 89.0524) (width 0.2) (layer "F.Cu") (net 2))
 (via (at 73.3744 89.0524) (size 0.6) (drill 0.3) (layers "F.Cu" "B.Cu") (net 2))
 (segment (start 78.545 71.425) (end 75.53 74.44) (width 0.2) (layer "B.Cu") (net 2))
 (segment (start 75.53 86.8968) (end 73.3744 89.0524) (width 0.2) (layer "B.Cu") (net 2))
 (segment (start 75.53 89.0524) (end 73.3744 89.0524) (width 0.2) (layer "B.Cu") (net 2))
 (segment (start 73.3744 89.0524) (end 75.53 89.0524) (width 0.2) (layer "B.Cu") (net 2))
 (segment (start 75.53 74.44) (end 75.53 86.8968) (width 0.2) (layer "B.Cu") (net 2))
 (segment (start 76.005 71.425) (end 74.18 73.25) (width 0.2) (layer "F.Cu") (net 17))
 (segment (start 74.18 73.25) (end 60.54 73.25) (width 0.2) (layer "F.Cu") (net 17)))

